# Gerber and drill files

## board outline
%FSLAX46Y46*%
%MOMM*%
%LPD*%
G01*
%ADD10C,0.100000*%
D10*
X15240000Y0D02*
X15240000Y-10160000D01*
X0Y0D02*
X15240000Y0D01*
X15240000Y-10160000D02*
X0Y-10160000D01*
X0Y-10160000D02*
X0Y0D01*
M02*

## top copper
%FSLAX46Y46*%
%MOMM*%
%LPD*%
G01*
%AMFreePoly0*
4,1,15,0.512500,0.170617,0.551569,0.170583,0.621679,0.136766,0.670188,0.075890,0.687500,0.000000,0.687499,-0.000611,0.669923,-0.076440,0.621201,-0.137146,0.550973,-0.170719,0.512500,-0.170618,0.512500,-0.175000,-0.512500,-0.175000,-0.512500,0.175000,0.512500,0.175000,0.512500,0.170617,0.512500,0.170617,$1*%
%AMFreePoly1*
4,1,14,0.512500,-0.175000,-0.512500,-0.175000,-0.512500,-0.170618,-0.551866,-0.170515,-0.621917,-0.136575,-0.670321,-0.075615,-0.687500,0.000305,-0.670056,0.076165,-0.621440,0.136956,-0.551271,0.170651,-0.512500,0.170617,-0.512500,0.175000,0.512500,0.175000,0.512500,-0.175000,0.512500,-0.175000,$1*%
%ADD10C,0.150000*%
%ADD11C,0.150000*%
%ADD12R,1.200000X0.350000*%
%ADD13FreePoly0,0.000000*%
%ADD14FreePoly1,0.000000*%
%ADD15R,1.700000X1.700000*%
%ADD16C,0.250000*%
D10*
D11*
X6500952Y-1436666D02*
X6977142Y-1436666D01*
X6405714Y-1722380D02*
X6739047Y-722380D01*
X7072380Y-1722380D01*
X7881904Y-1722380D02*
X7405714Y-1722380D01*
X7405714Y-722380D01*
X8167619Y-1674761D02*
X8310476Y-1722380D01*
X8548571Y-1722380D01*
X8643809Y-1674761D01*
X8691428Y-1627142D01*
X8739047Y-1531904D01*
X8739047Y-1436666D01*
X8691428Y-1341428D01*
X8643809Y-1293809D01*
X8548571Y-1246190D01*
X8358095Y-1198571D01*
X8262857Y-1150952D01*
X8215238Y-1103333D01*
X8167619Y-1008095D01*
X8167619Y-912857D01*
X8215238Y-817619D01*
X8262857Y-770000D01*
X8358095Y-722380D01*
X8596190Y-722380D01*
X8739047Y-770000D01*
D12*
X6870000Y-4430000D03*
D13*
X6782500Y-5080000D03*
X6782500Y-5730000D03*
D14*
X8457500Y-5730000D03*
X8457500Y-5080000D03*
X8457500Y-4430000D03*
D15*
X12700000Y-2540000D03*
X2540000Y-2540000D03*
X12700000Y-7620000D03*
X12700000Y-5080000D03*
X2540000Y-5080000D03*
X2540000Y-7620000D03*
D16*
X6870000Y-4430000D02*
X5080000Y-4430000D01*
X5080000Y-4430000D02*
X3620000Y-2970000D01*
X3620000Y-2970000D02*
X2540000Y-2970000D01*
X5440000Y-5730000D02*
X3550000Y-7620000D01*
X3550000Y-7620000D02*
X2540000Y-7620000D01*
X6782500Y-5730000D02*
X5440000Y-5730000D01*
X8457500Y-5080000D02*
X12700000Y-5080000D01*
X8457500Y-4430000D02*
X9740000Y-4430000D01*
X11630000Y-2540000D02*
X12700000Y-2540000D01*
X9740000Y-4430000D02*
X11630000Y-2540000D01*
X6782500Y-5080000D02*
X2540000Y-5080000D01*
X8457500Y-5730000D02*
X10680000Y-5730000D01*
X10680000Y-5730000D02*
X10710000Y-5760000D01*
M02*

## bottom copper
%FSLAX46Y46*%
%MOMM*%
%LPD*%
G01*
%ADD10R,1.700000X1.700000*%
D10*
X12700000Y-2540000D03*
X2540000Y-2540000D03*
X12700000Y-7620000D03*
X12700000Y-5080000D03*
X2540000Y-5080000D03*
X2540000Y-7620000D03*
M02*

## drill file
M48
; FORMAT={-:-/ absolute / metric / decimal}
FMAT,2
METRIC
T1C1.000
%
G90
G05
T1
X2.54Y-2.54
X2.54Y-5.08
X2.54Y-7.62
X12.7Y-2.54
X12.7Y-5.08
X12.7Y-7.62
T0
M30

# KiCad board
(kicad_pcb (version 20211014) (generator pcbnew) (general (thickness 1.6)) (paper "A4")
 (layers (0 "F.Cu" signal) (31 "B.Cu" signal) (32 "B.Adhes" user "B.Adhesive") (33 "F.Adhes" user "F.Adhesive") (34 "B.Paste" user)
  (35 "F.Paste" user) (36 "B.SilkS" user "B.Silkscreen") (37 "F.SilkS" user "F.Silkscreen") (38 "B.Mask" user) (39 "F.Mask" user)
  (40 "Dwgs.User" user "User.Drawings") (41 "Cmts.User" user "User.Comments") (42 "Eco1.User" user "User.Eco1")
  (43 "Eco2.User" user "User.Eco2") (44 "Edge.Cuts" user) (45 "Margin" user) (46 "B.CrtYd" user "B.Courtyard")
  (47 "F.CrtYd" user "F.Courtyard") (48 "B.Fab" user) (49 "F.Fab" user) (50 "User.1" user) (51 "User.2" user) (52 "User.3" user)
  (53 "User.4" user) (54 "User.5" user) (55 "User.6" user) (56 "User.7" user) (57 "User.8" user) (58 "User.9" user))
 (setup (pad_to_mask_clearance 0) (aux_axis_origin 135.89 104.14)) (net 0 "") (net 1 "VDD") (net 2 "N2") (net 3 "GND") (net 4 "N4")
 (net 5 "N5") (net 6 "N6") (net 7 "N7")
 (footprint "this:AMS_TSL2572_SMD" (layer "F.Cu") (at 143.51 109.22)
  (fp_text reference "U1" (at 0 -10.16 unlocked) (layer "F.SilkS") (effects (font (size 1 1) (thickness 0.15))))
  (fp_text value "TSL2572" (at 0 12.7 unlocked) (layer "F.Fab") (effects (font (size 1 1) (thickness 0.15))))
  (pad "1" smd rect (at -0.75 -0.65) (size 1.2 0.35) (layers "F.Cu" "F.Paste" "F.Mask") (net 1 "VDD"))
  (pad "2" smd custom (at -0.8375 0) (size 1.025 0.35) (layers "F.Cu" "F.Paste" "F.Mask") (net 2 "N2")
   (options (clearance outline) (anchor rect)) (primitives))
  (pad "3" smd custom (at -0.8375 0.65) (size 1.025 0.35) (layers "F.Cu" "F.Paste" "F.Mask") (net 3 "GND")
   (options (clearance outline) (anchor rect)) (primitives))
  (pad "4" smd custom (at 0.8375 0.65) (size 1.025 0.35) (layers "F.Cu" "F.Paste" "F.Mask") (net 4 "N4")
   (options (clearance outline) (anchor rect)) (primitives))
  (pad "5" smd custom (at 0.8375 0) (size 1.025 0.35) (layers "F.Cu" "F.Paste" "F.Mask") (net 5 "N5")
   (options (clearance outline) (anchor rect)) (primitives))
  (pad "6" smd custom (at 0.8375 -0.65) (size 1.025 0.35) (layers "F.Cu" "F.Paste" "F.Mask") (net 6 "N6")
   (options (clearance outline) (anchor rect)) (primitives)))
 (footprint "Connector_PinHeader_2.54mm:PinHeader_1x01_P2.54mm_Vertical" (layer "B.Cu") (at 148.59 106.68 180)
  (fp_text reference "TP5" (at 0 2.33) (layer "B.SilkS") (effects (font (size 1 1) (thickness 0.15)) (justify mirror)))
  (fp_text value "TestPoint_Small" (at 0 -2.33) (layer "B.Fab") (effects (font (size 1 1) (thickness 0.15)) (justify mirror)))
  (pad "1" thru_hole rect (at 0 0 180) (size 1.7 1.7) (drill 1) (layers *.Cu *.Mask) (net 6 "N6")))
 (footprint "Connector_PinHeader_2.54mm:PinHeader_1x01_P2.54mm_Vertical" (layer "B.Cu") (at 138.43 106.68 180)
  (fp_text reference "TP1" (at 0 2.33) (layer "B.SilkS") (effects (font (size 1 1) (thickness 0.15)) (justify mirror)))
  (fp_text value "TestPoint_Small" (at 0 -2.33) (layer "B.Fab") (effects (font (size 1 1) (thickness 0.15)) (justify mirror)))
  (pad "1" thru_hole rect (at 0 0 180) (size 1.7 1.7) (drill 1) (layers *.Cu *.Mask) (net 1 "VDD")))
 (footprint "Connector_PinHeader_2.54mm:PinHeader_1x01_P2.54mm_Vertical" (layer "B.Cu") (at 148.59 111.76 180)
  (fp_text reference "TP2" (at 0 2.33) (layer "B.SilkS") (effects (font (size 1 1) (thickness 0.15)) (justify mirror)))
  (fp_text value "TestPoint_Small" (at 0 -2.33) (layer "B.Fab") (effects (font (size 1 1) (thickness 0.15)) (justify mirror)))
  (pad "1" thru_hole rect (at 0 0 180) (size 1.7 1.7) (drill 1) (layers *.Cu *.Mask) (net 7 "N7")))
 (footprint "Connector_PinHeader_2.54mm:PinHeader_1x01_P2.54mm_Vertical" (layer "B.Cu") (at 148.59 109.22 180)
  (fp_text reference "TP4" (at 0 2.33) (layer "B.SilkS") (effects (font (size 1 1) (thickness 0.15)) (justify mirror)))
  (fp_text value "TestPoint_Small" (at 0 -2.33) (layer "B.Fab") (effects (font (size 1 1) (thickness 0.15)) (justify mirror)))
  (pad "1" thru_hole rect (at 0 0 180) (size 1.7 1.7) (drill 1) (layers *.Cu *.Mask) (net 5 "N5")))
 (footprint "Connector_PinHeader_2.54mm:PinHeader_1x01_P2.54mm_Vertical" (layer "B.Cu") (at 138.43 109.22 180)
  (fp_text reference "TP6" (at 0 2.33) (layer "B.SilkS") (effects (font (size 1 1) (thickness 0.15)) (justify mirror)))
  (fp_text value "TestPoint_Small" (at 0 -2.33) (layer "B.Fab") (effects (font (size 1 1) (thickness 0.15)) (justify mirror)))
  (pad "1" thru_hole rect (at 0 0 180) (size 1.7 1.7) (drill 1) (layers *.Cu *.Mask) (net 2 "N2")))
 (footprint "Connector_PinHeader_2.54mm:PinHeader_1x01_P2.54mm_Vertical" (layer "B.Cu") (at 138.43 111.76 180)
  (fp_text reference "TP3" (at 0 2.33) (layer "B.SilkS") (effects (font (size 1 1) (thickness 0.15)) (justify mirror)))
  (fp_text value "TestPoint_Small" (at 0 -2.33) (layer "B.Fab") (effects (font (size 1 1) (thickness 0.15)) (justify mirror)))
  (pad "1" thru_hole rect (at 0 0 180) (size 1.7 1.7) (drill 1) (layers *.Cu *.Mask) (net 3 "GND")))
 (gr_line (start 151.13 104.14) (end 151.13 114.3) (layer "Edge.Cuts") (width 0.1))
 (gr_line (start 135.89 104.14) (end 151.13 104.14) (layer "Edge.Cuts") (width 0.1))
 (gr_line (start 151.13 114.3) (end 135.89 114.3) (layer "Edge.Cuts") (width 0.1))
 (gr_line (start 135.89 114.3) (end 135.89 104.14) (layer "Edge.Cuts") (width 0.1))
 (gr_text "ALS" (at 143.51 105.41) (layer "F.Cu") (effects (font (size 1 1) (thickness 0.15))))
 (segment (start 142.76 108.57) (end 140.97 108.57) (width 0.25) (layer "F.Cu") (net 1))
 (segment (start 140.97 108.57) (end 139.51 107.11) (width 0.25) (layer "F.Cu") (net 1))
 (segment (start 139.51 107.11) (end 138.43 107.11) (width 0.25) (layer "F.Cu") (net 1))
 (segment (start 141.33 109.87) (end 139.44 111.76) (width 0.25) (layer "F.Cu") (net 3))
 (segment (start 139.44 111.76) (end 138.43 111.76) (width 0.25) (layer "F.Cu") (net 3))
 (segment (start 142.6725 109.87) (end 141.33 109.87) (width 0.25) (layer "F.Cu") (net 3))
 (segment (start 144.3475 109.22) (end 148.59 109.22) (width 0.25) (layer "F.Cu") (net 5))
 (segment (start 144.3475 108.57) (end 145.63 108.57) (width 0.25) (layer "F.Cu") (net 6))
 (segment (start 147.52 106.68) (end 148.59 106.68) (width 0.25) (layer "F.Cu") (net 6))
 (segment (start 145.63 108.57) (end 147.52 106.68) (width 0.25) (layer "F.Cu") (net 6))
 (segment (start 142.6725 109.22) (end 138.43 109.22) (width 0.25) (layer "F.Cu") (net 2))
 (segment (start 144.3475 109.87) (end 146.57 109.87) (width 0.25) (layer "F.Cu") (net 4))
 (segment (start 146.57 109.87) (end 146.6 109.9) (width 0.25) (layer "F.Cu") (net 4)))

